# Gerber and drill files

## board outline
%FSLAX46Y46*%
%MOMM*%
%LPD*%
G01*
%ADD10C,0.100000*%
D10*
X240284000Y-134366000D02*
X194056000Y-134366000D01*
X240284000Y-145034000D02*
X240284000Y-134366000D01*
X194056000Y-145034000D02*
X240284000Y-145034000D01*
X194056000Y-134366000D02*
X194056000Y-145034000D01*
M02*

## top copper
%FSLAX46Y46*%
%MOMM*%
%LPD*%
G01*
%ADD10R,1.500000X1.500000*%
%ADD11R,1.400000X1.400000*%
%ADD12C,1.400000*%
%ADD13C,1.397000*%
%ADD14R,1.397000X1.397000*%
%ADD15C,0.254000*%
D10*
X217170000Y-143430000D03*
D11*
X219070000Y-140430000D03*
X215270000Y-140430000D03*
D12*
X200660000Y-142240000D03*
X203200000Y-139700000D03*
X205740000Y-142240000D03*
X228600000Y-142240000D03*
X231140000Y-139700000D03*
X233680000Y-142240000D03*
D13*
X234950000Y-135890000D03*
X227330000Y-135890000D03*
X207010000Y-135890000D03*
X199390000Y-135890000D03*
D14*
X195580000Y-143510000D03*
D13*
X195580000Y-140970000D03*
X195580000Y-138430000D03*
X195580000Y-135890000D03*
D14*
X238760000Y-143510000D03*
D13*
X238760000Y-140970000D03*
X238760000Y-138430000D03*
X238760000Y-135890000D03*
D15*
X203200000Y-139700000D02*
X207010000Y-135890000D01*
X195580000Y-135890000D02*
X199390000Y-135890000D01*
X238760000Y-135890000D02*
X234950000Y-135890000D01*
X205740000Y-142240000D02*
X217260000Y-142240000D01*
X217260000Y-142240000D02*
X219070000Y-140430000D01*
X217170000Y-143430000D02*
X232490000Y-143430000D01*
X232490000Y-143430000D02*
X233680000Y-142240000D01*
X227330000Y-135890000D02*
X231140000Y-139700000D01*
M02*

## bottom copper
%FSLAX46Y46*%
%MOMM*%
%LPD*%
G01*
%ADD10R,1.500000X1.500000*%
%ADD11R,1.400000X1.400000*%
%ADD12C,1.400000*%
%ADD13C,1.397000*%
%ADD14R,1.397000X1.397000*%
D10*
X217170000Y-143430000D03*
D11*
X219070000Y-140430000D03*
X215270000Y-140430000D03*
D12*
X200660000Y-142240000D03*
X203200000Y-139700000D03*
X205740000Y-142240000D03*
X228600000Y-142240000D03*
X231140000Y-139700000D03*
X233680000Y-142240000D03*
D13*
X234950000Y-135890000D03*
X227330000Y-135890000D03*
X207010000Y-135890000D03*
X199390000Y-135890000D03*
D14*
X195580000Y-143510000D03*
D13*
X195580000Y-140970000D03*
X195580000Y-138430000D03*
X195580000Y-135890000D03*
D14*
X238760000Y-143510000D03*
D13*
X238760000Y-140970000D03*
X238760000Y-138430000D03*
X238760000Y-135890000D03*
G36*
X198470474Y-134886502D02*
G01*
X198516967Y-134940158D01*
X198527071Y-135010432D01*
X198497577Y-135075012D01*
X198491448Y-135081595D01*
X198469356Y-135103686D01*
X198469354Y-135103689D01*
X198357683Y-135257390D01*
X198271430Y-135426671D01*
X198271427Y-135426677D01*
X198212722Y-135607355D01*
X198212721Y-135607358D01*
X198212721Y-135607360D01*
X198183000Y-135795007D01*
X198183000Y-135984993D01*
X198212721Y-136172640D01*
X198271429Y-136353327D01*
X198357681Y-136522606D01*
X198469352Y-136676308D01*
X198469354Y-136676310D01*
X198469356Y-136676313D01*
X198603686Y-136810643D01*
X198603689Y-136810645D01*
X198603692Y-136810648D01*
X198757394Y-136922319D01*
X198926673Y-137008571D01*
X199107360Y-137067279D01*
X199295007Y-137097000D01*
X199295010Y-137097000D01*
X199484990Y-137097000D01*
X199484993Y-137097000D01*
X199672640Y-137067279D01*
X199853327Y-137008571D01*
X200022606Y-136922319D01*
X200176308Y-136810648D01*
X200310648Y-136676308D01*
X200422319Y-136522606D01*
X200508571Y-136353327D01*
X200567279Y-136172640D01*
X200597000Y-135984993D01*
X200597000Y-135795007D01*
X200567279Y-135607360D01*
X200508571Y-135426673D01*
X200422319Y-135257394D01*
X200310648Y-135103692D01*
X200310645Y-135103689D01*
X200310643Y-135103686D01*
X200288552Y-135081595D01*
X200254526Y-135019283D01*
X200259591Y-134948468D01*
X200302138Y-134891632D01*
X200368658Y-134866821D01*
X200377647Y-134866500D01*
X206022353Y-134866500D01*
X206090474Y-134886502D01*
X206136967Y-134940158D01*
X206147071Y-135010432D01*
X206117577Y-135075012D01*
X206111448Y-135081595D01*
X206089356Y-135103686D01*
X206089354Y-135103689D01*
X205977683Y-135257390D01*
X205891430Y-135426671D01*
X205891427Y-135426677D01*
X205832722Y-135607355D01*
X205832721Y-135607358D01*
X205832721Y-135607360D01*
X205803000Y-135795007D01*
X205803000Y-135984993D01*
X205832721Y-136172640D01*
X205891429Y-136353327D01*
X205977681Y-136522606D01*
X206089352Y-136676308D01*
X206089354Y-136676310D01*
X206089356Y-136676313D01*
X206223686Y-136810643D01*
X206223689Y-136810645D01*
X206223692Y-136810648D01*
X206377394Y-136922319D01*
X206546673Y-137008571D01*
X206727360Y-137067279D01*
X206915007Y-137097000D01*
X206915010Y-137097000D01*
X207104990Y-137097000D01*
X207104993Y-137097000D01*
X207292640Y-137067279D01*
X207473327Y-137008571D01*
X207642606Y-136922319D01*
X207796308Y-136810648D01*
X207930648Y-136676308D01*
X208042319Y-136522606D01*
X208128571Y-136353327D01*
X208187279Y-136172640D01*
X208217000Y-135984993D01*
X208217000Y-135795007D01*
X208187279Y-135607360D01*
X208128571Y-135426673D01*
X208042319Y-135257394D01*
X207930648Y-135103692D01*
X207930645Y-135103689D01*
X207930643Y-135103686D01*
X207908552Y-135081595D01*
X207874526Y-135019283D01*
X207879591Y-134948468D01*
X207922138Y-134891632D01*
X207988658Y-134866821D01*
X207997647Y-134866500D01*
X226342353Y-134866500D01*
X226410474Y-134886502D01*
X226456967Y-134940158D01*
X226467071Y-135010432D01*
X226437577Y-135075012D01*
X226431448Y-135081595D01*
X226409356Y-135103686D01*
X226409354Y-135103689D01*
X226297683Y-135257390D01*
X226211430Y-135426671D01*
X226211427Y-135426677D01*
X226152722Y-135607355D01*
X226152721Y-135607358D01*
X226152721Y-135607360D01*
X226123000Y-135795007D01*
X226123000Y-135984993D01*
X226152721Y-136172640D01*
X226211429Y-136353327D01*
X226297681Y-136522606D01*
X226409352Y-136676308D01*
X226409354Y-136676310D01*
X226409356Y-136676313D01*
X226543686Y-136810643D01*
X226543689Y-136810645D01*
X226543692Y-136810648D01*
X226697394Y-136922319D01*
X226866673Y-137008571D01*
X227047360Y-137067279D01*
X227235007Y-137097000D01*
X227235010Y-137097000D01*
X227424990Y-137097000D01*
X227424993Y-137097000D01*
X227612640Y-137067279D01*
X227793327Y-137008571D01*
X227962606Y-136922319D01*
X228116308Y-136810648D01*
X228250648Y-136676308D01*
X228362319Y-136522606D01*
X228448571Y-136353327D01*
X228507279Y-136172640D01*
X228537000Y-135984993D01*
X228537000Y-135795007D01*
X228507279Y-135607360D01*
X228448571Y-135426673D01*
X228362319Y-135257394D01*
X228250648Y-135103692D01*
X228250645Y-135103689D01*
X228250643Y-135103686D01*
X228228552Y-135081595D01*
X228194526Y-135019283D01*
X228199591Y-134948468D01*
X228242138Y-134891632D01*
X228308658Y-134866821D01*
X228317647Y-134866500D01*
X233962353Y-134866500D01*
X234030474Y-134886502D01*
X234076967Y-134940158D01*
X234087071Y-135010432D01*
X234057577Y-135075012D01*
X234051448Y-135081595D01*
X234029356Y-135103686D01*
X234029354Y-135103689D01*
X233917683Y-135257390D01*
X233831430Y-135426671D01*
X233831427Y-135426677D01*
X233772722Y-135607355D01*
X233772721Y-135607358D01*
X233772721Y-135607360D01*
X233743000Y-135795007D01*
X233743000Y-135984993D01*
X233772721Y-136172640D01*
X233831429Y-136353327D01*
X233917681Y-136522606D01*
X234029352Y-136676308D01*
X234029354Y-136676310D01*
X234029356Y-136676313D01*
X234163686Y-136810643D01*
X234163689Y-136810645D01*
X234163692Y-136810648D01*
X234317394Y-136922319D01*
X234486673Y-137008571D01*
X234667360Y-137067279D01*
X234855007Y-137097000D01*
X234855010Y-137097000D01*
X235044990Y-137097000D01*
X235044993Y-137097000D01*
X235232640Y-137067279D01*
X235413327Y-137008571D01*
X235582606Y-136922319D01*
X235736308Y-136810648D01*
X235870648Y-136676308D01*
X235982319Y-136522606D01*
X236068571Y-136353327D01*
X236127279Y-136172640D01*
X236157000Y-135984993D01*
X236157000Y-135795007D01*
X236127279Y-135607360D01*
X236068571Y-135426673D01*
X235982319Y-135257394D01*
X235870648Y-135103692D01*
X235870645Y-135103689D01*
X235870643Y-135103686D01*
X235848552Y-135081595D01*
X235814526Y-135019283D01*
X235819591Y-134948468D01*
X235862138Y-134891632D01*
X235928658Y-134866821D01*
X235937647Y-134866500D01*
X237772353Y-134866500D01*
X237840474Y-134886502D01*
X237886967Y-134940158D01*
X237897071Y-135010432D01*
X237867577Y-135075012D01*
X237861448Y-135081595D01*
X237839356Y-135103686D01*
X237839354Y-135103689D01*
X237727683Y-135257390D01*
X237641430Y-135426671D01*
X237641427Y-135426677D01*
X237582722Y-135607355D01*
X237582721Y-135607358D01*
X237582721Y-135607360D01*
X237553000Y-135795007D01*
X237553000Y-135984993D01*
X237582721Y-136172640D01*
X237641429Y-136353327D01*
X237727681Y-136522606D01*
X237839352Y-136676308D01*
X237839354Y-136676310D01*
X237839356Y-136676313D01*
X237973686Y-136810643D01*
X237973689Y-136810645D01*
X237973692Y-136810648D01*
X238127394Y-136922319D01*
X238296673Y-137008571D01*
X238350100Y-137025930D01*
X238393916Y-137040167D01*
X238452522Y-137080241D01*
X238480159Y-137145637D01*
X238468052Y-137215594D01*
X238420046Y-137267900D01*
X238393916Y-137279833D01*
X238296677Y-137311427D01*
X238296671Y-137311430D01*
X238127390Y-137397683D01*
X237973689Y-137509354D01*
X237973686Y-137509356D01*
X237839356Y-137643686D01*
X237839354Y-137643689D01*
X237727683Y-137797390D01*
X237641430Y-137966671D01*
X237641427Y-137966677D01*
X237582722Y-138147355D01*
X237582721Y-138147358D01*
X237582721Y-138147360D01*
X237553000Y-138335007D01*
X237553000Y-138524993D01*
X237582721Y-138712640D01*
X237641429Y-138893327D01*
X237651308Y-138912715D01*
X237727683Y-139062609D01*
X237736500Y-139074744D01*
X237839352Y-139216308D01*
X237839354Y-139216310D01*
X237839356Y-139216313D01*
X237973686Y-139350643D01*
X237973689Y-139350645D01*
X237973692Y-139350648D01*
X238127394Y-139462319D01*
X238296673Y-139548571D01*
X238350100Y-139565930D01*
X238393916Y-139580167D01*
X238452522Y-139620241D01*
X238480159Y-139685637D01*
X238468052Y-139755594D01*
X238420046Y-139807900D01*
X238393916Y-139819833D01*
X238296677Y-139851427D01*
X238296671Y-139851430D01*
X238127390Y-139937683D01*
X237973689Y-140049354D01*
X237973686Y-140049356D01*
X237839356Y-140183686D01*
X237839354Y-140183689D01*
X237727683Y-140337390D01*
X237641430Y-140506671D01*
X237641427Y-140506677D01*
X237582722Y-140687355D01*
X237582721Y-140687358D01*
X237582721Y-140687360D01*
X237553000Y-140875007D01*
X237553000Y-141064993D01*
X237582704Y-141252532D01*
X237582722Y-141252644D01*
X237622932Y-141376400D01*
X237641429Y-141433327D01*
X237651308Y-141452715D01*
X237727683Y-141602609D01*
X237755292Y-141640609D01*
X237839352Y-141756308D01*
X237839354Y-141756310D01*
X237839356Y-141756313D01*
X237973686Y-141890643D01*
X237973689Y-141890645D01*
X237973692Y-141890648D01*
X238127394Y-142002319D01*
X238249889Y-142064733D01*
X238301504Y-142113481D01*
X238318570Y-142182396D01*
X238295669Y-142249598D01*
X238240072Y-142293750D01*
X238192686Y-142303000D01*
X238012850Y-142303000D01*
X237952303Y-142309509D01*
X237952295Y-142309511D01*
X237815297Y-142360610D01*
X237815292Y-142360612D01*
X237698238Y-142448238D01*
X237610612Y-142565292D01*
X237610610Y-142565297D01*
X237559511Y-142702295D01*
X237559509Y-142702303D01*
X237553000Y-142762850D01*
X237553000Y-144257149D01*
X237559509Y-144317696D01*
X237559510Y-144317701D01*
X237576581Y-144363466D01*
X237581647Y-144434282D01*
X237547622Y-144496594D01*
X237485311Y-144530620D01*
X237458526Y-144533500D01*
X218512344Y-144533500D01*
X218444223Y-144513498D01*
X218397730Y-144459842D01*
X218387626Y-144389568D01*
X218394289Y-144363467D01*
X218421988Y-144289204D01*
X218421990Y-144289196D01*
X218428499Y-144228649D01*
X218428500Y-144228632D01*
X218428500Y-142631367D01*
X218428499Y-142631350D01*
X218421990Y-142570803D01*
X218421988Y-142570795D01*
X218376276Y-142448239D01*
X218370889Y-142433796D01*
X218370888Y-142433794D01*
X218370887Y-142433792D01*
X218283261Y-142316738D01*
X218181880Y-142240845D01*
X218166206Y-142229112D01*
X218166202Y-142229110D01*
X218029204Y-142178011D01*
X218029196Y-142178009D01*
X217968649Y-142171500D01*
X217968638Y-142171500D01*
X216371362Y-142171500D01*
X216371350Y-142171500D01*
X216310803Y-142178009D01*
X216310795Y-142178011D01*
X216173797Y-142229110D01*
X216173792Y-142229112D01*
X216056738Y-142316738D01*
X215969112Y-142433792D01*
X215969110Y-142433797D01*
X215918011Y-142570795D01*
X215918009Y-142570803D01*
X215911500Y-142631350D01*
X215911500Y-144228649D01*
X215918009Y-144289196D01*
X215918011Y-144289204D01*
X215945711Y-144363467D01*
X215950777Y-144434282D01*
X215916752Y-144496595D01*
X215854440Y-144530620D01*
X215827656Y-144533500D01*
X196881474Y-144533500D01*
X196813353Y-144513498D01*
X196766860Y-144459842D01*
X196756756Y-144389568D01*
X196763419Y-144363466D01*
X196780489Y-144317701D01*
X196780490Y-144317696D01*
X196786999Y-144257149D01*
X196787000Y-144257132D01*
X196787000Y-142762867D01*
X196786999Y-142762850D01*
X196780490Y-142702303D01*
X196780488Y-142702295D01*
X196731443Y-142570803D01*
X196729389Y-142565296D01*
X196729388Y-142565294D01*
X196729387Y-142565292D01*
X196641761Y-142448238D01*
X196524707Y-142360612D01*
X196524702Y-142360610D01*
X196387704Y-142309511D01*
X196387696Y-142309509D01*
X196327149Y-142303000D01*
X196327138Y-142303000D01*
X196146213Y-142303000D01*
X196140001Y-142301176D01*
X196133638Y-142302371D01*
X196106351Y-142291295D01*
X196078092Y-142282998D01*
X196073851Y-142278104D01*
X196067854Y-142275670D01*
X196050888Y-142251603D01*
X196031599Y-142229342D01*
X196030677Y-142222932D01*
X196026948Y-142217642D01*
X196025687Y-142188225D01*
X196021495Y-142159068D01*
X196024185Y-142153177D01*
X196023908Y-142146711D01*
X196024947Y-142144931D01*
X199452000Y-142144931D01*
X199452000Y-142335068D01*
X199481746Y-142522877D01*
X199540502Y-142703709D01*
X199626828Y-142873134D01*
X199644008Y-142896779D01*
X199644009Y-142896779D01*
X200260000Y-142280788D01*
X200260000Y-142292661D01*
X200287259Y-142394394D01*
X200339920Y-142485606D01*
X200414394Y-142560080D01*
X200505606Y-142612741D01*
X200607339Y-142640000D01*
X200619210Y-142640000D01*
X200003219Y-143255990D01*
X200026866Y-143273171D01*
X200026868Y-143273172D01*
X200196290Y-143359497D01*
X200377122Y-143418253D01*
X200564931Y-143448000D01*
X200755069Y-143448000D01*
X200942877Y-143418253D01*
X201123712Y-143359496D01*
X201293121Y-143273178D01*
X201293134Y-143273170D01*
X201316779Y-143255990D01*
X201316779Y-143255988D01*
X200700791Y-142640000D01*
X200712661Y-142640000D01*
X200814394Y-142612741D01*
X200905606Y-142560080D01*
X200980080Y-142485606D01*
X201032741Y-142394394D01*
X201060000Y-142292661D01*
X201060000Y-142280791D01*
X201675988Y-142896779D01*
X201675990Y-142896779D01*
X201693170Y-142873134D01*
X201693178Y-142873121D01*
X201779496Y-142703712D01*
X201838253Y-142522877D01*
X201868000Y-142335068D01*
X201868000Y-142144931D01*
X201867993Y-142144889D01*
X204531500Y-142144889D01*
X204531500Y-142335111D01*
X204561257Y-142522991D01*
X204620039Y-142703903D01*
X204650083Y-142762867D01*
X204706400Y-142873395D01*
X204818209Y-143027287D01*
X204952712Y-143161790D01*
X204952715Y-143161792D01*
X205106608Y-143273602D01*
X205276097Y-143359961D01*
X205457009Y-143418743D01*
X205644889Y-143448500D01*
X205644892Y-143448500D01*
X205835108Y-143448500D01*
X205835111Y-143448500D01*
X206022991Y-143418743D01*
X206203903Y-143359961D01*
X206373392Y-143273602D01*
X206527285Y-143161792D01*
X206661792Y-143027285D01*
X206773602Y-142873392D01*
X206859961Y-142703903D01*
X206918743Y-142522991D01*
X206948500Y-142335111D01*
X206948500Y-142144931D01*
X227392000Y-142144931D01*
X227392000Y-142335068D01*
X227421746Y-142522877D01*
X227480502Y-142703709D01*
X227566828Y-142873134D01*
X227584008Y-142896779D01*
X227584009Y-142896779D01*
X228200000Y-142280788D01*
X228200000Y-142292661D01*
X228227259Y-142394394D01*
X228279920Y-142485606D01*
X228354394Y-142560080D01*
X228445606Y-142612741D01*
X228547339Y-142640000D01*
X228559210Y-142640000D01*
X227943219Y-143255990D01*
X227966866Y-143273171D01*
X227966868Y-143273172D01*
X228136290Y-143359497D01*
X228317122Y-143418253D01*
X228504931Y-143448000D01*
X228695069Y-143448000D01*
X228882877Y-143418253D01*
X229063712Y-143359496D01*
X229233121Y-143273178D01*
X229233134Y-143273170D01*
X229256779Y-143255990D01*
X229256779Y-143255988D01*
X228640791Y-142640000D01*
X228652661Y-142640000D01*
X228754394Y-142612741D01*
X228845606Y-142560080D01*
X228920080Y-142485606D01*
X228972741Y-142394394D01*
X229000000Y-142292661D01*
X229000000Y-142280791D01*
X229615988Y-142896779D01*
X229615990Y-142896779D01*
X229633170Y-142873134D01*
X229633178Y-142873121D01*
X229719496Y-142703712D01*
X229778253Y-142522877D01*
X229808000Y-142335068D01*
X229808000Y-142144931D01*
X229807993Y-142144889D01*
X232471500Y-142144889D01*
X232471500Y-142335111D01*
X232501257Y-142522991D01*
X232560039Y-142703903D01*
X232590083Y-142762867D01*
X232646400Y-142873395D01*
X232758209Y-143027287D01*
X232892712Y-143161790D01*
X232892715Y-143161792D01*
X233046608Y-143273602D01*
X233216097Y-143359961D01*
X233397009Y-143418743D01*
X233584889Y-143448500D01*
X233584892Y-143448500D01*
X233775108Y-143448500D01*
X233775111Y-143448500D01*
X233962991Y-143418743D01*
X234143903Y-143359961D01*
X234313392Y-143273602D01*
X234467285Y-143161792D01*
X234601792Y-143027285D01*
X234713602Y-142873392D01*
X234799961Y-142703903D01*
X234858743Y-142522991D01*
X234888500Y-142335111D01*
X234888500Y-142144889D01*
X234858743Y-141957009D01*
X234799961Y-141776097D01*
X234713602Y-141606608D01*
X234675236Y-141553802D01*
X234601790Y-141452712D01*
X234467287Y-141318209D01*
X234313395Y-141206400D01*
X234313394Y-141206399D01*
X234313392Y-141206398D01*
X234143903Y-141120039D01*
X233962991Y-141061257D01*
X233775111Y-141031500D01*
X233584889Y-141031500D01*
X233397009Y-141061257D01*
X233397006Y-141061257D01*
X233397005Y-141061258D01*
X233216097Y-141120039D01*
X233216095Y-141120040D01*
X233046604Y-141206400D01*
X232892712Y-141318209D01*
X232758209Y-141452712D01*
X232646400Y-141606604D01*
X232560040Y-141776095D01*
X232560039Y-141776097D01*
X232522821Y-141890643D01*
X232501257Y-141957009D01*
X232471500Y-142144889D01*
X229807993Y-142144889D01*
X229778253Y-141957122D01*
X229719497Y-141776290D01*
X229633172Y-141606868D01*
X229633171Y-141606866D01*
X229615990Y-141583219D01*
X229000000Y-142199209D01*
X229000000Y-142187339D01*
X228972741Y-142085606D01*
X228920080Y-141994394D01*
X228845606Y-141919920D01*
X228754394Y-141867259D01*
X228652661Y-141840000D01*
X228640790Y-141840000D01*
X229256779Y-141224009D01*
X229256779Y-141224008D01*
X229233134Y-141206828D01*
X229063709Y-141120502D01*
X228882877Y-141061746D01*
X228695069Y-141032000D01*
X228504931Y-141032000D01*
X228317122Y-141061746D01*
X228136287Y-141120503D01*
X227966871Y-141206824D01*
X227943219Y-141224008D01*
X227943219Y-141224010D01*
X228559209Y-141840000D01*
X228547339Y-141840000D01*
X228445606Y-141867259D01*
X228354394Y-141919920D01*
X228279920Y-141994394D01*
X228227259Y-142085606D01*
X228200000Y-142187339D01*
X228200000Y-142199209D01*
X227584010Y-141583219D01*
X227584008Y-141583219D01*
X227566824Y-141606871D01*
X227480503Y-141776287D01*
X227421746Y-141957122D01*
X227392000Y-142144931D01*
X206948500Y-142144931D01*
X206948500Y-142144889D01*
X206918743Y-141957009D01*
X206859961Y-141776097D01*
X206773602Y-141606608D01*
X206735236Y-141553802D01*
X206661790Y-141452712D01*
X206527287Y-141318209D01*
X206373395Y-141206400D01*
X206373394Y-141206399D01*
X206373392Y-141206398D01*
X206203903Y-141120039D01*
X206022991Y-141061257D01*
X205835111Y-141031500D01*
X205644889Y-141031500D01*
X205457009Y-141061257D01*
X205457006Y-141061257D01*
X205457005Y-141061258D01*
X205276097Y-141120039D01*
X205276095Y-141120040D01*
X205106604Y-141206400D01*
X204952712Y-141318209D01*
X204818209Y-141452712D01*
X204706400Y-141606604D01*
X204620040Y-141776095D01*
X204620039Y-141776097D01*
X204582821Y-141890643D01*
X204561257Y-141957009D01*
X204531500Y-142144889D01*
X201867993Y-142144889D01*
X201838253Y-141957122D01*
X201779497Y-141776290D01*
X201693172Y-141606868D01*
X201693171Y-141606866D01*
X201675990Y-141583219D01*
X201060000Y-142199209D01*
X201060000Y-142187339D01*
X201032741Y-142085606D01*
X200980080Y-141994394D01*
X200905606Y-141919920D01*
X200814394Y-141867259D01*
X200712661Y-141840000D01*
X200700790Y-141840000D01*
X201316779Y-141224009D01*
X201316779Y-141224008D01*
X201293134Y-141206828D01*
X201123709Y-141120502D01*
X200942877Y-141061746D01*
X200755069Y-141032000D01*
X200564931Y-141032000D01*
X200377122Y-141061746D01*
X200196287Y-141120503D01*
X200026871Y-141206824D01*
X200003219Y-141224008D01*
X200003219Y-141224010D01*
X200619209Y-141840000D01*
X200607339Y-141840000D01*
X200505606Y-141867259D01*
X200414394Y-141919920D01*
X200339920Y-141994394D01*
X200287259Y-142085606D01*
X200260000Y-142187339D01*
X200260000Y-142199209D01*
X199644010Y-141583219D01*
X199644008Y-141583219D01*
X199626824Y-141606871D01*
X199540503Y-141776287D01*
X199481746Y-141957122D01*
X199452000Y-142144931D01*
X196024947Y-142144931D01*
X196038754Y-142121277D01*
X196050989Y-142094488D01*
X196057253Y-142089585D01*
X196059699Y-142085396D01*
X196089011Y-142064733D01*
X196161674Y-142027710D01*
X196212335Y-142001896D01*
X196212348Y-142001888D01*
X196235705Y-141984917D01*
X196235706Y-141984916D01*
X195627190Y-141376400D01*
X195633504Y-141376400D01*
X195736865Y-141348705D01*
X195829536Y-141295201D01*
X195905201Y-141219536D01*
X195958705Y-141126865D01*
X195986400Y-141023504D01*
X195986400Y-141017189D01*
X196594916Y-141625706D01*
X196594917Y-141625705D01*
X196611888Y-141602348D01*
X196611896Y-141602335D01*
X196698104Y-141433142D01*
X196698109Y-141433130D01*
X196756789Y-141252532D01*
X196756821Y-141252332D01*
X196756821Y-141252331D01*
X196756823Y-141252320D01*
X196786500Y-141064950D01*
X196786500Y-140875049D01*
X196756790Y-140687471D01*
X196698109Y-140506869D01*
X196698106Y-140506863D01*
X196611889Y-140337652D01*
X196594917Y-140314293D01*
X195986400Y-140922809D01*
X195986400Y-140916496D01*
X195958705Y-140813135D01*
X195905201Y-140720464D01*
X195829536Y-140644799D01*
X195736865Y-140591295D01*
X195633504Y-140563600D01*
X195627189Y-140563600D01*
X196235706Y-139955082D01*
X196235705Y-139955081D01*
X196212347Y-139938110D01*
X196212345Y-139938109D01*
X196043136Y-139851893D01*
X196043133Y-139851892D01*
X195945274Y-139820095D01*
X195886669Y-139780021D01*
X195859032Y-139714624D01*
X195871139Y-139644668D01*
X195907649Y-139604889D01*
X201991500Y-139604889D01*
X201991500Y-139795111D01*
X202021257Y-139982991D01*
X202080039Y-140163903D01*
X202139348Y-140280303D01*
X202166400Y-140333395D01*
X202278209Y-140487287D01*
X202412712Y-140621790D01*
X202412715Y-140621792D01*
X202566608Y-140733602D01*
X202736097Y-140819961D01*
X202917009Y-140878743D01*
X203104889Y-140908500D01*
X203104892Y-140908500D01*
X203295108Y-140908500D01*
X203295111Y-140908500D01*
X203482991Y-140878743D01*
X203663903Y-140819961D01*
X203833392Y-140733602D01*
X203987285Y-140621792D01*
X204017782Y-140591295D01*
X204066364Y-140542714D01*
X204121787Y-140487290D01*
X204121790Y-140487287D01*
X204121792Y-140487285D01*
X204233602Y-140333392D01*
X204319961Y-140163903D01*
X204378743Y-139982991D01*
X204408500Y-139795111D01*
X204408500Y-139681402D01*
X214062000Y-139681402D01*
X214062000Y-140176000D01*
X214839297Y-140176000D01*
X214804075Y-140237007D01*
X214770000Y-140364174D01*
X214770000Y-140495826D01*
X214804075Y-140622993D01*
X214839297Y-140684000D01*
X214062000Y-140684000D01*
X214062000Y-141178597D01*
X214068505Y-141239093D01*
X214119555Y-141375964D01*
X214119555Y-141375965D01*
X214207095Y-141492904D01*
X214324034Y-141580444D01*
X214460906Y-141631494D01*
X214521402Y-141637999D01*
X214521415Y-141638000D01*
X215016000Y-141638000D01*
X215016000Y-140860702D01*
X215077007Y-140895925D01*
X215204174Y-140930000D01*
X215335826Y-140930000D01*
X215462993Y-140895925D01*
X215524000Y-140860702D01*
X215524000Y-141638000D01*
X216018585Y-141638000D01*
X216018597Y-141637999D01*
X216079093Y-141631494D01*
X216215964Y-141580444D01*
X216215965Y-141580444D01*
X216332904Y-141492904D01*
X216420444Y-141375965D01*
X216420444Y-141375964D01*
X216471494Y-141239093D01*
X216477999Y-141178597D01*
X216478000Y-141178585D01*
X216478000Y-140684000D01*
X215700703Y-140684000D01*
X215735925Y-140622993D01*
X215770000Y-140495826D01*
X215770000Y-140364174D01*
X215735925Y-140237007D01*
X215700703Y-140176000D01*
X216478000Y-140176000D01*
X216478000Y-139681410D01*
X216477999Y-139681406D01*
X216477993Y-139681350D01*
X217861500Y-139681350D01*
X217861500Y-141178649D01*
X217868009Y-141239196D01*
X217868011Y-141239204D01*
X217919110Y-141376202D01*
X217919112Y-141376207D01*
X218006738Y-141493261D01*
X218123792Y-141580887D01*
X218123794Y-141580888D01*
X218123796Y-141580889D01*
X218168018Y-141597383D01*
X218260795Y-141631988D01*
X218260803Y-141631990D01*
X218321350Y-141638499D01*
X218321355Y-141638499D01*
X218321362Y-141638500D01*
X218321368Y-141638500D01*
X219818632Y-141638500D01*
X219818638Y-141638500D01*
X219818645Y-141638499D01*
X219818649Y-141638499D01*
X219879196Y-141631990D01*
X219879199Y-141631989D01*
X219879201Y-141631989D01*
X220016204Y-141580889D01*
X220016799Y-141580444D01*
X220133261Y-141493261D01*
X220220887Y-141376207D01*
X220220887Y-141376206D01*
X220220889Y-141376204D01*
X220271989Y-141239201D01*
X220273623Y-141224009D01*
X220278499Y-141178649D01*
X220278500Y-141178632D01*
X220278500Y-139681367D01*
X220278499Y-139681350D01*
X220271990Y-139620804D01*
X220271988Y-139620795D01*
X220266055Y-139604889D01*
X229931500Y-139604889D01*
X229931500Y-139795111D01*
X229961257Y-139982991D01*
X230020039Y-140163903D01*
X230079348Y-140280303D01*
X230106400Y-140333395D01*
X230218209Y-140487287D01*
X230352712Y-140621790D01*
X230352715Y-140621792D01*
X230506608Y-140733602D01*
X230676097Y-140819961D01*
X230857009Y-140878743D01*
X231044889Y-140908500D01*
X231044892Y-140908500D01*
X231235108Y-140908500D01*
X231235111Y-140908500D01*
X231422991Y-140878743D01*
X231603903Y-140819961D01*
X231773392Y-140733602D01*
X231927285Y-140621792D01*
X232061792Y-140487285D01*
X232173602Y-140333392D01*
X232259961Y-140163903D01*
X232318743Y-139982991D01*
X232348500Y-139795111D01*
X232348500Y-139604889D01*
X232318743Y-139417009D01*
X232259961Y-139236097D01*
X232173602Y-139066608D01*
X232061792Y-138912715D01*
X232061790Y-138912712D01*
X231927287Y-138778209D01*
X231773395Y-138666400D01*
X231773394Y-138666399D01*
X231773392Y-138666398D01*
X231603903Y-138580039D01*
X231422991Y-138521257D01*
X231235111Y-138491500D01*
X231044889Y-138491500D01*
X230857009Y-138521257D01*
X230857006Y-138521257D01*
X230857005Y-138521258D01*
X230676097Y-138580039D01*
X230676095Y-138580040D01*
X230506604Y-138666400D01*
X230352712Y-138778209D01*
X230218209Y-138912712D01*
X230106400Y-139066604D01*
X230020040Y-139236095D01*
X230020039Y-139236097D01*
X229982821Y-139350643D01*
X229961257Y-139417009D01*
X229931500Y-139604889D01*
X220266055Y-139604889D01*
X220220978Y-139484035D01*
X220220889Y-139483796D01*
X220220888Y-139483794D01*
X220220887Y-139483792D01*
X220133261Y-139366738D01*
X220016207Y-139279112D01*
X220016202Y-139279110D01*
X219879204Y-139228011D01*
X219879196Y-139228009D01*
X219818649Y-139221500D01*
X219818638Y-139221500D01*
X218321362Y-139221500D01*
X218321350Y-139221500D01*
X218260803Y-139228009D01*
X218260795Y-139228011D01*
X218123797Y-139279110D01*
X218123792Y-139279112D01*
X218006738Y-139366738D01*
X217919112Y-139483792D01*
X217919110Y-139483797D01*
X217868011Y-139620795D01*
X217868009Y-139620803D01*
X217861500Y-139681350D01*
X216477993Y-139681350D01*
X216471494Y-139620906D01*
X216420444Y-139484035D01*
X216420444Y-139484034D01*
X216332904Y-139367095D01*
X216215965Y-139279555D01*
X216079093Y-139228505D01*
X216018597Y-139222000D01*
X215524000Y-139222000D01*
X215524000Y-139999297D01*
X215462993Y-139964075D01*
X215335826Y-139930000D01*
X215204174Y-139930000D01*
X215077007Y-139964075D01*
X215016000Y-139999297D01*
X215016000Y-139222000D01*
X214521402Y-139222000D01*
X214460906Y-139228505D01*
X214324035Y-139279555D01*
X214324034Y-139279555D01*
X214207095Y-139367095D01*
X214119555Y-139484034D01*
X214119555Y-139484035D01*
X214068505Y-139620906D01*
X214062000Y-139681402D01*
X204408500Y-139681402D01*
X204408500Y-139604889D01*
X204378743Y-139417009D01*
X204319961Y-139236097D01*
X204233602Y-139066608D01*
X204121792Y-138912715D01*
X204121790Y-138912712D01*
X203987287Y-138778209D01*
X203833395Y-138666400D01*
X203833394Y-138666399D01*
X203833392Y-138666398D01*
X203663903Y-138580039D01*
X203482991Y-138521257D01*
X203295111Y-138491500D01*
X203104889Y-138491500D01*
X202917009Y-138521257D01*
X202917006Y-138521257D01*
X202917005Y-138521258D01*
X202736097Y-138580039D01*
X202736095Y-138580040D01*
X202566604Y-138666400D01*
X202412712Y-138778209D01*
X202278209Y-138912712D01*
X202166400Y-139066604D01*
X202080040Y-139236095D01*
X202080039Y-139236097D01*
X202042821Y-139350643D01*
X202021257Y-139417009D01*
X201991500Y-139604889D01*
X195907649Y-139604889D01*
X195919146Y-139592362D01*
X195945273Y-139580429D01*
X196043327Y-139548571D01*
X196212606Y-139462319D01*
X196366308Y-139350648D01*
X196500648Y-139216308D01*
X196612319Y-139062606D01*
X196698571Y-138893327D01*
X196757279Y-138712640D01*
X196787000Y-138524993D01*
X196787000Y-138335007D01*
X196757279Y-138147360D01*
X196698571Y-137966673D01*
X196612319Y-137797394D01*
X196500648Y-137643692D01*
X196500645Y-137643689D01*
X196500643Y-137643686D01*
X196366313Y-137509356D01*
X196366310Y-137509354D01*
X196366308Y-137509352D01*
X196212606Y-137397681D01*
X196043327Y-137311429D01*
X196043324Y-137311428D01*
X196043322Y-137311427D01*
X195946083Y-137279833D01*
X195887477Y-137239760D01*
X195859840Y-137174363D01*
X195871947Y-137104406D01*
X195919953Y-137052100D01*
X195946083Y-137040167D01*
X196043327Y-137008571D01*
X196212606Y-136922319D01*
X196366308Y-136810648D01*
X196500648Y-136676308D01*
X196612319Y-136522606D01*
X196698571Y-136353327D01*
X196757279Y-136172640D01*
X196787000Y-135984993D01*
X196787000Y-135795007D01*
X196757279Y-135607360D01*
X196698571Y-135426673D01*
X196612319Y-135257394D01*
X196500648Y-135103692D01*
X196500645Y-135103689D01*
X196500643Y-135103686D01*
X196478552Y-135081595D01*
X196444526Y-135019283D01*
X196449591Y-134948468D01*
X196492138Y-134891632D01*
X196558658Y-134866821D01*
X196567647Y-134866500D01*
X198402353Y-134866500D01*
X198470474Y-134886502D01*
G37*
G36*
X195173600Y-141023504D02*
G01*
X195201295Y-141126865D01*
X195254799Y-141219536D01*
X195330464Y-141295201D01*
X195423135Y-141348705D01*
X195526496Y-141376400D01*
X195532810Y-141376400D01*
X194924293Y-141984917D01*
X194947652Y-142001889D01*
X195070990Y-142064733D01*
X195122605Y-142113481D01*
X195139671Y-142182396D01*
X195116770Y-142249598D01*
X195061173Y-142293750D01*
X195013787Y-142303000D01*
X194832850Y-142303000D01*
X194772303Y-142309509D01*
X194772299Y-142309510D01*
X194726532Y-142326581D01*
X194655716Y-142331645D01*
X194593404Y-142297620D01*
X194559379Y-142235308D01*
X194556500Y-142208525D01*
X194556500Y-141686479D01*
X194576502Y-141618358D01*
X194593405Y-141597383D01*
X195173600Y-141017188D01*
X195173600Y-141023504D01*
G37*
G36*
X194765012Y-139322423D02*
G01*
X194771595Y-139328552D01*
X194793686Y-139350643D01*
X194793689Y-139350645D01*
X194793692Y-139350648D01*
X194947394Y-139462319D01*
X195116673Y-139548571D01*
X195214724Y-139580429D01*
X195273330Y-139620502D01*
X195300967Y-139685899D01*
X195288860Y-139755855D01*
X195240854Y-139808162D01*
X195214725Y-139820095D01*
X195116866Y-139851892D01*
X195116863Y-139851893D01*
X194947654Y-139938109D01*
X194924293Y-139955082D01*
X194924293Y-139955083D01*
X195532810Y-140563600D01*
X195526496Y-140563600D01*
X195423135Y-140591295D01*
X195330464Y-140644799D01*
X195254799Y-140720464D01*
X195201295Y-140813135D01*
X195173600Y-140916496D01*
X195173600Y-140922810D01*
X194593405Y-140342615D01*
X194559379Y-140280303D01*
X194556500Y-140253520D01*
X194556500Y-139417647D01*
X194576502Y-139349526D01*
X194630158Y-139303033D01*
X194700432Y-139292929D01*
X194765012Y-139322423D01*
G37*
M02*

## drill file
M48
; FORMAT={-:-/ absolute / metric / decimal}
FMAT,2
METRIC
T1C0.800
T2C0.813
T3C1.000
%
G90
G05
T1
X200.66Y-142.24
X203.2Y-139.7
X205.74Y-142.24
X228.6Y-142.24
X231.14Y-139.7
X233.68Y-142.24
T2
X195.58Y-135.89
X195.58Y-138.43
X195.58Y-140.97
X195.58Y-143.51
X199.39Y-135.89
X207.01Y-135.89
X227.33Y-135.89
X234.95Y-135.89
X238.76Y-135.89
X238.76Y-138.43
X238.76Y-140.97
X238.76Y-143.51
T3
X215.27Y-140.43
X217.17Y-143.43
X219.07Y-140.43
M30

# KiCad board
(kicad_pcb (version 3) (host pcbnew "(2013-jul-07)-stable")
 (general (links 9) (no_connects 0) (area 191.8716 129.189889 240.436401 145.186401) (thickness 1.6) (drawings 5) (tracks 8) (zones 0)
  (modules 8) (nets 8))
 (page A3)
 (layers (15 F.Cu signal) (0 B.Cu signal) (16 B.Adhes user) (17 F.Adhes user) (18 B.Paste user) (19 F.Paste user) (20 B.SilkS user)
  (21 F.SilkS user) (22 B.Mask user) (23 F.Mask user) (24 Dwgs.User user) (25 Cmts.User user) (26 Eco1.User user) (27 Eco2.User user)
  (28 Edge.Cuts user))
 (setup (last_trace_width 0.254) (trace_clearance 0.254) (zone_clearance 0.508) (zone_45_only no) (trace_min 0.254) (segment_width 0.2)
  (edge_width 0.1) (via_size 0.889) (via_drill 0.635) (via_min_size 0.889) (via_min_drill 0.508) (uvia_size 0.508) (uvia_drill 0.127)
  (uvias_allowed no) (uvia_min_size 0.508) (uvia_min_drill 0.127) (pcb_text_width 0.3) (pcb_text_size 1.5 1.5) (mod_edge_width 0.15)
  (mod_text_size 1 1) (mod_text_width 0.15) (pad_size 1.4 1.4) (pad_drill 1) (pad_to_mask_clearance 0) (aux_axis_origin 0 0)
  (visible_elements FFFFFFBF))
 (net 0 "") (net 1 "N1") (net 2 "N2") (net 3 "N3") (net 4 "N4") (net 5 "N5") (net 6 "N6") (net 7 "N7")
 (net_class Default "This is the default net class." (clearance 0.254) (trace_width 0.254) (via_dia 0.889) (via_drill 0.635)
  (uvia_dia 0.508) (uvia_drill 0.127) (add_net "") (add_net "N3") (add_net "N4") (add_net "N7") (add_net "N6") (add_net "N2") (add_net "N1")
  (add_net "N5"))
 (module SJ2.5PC (layer F.Cu) (at 217.17 138.43 270)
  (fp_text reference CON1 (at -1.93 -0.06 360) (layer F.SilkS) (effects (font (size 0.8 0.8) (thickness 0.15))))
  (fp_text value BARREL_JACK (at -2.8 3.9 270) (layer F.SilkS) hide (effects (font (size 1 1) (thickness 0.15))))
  (pad 3 thru_hole rect (at 5 0 270) (size 1.5 1.5) (drill 1) (layers *.Cu *.Mask F.SilkS) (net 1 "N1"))
  (pad 2 thru_hole rect (at 2 -1.9 270) (size 1.4 1.4) (drill 1) (layers *.Cu *.Mask F.SilkS) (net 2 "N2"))
  (pad 1 thru_hole rect (at 2 1.9 270) (size 1.4 1.4) (drill 1) (layers *.Cu *.Mask F.SilkS) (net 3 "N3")))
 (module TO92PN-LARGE (layer F.Cu) (at 203.2 139.7 180)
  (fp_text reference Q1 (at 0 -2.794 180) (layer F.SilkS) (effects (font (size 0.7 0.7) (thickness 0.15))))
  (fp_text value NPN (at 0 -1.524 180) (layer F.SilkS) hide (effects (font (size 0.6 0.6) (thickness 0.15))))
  (pad 1 thru_hole circle (at 2.54 -2.54 180) (size 1.4 1.4) (drill 0.8) (layers *.Cu *.Mask F.SilkS) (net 3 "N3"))
  (pad 2 thru_hole circle (at 0 0 180) (size 1.4 1.4) (drill 0.8) (layers *.Cu *.Mask F.SilkS) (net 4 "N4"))
  (pad 3 thru_hole circle (at -2.54 -2.54 180) (size 1.4 1.4) (drill 0.8) (layers *.Cu *.Mask F.SilkS) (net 2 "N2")))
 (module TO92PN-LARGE (layer F.Cu) (at 231.14 139.7 180)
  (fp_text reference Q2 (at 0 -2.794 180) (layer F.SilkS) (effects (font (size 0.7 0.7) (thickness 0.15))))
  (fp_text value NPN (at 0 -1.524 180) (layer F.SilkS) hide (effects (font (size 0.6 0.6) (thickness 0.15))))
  (pad 1 thru_hole circle (at 2.54 -2.54 180) (size 1.4 1.4) (drill 0.8) (layers *.Cu *.Mask F.SilkS) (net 3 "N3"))
  (pad 2 thru_hole circle (at 0 0 180) (size 1.4 1.4) (drill 0.8) (layers *.Cu *.Mask F.SilkS) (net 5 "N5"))
  (pad 3 thru_hole circle (at -2.54 -2.54 180) (size 1.4 1.4) (drill 0.8) (layers *.Cu *.Mask F.SilkS) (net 1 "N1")))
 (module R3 (layer F.Cu) (at 231.14 135.89 180) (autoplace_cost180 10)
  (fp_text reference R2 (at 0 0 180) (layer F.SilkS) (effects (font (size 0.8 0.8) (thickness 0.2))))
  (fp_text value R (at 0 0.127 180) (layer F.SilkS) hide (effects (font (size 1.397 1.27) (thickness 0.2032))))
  (pad 1 thru_hole circle (at -3.81 0 180) (size 1.397 1.397) (drill 0.8128) (layers *.Cu *.Mask F.SilkS) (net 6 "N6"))
  (pad 2 thru_hole circle (at 3.81 0 180) (size 1.397 1.397) (drill 0.8128) (layers *.Cu *.Mask F.SilkS) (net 5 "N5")))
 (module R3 (layer F.Cu) (at 203.2 135.89 180) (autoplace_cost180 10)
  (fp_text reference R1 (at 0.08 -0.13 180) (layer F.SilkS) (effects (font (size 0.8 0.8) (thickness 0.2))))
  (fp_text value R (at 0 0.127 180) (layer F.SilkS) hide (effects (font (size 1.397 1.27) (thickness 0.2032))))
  (pad 1 thru_hole circle (at -3.81 0 180) (size 1.397 1.397) (drill 0.8128) (layers *.Cu *.Mask F.SilkS) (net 4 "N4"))
  (pad 2 thru_hole circle (at 3.81 0 180) (size 1.397 1.397) (drill 0.8128) (layers *.Cu *.Mask F.SilkS) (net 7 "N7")))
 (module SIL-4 (layer F.Cu) (at 195.58 139.7 90)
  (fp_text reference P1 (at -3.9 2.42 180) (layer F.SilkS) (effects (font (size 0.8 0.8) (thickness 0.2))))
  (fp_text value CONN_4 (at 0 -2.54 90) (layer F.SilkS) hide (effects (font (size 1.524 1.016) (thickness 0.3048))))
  (pad 1 thru_hole rect (at -3.81 0 90) (size 1.397 1.397) (drill 0.8128) (layers *.Cu *.Mask F.SilkS))
  (pad 2 thru_hole circle (at -1.27 0 90) (size 1.397 1.397) (drill 0.8128) (layers *.Cu *.Mask F.SilkS) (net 3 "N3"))
  (pad 3 thru_hole circle (at 1.27 0 90) (size 1.397 1.397) (drill 0.8128) (layers *.Cu *.Mask F.SilkS))
  (pad 4 thru_hole circle (at 3.81 0 90) (size 1.397 1.397) (drill 0.8128) (layers *.Cu *.Mask F.SilkS) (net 7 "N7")))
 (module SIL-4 (layer F.Cu) (at 238.76 139.7 90)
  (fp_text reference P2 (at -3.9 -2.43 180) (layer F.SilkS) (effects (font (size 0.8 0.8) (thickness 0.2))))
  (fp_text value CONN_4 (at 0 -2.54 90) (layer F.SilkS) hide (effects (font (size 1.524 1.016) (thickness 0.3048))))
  (pad 1 thru_hole rect (at -3.81 0 90) (size 1.397 1.397) (drill 0.8128) (layers *.Cu *.Mask F.SilkS))
  (pad 2 thru_hole circle (at -1.27 0 90) (size 1.397 1.397) (drill 0.8128) (layers *.Cu *.Mask F.SilkS))
  (pad 3 thru_hole circle (at 1.27 0 90) (size 1.397 1.397) (drill 0.8128) (layers *.Cu *.Mask F.SilkS))
  (pad 4 thru_hole circle (at 3.81 0 90) (size 1.397 1.397) (drill 0.8128) (layers *.Cu *.Mask F.SilkS) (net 6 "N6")))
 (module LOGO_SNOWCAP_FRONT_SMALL (layer F.Cu) (at 210.82 139.446 90)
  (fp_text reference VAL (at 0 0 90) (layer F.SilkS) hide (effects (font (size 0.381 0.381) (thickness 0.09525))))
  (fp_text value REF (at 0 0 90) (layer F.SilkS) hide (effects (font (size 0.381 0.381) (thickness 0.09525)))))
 (gr_line (start 240.284 134.366) (end 194.056 134.366) (angle 90) (layer Edge.Cuts) (width 0.1))
 (gr_line (start 240.284 145.034) (end 240.284 134.366) (angle 90) (layer Edge.Cuts) (width 0.1))
 (gr_line (start 194.056 145.034) (end 240.284 145.034) (angle 90) (layer Edge.Cuts) (width 0.1))
 (gr_line (start 194.056 134.366) (end 194.056 145.034) (angle 90) (layer Edge.Cuts) (width 0.1))
 (segment (start 203.2 139.7) (end 207.01 135.89) (width 0.254) (layer F.Cu) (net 4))
 (segment (start 195.58 135.89) (end 199.39 135.89) (width 0.254) (layer F.Cu) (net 7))
 (segment (start 238.76 135.89) (end 234.95 135.89) (width 0.254) (layer F.Cu) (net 6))
 (segment (start 205.74 142.24) (end 217.26 142.24) (width 0.254) (layer F.Cu) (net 2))
 (segment (start 217.26 142.24) (end 219.07 140.43) (width 0.254) (layer F.Cu) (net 2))
 (segment (start 217.17 143.43) (end 232.49 143.43) (width 0.254) (layer F.Cu) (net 1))
 (segment (start 232.49 143.43) (end 233.68 142.24) (width 0.254) (layer F.Cu) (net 1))
 (segment (start 227.33 135.89) (end 231.14 139.7) (width 0.254) (layer F.Cu) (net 5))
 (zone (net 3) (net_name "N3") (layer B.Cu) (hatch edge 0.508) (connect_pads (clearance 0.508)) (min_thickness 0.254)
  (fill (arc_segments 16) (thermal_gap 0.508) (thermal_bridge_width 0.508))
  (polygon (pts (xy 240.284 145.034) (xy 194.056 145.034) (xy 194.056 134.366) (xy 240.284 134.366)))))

